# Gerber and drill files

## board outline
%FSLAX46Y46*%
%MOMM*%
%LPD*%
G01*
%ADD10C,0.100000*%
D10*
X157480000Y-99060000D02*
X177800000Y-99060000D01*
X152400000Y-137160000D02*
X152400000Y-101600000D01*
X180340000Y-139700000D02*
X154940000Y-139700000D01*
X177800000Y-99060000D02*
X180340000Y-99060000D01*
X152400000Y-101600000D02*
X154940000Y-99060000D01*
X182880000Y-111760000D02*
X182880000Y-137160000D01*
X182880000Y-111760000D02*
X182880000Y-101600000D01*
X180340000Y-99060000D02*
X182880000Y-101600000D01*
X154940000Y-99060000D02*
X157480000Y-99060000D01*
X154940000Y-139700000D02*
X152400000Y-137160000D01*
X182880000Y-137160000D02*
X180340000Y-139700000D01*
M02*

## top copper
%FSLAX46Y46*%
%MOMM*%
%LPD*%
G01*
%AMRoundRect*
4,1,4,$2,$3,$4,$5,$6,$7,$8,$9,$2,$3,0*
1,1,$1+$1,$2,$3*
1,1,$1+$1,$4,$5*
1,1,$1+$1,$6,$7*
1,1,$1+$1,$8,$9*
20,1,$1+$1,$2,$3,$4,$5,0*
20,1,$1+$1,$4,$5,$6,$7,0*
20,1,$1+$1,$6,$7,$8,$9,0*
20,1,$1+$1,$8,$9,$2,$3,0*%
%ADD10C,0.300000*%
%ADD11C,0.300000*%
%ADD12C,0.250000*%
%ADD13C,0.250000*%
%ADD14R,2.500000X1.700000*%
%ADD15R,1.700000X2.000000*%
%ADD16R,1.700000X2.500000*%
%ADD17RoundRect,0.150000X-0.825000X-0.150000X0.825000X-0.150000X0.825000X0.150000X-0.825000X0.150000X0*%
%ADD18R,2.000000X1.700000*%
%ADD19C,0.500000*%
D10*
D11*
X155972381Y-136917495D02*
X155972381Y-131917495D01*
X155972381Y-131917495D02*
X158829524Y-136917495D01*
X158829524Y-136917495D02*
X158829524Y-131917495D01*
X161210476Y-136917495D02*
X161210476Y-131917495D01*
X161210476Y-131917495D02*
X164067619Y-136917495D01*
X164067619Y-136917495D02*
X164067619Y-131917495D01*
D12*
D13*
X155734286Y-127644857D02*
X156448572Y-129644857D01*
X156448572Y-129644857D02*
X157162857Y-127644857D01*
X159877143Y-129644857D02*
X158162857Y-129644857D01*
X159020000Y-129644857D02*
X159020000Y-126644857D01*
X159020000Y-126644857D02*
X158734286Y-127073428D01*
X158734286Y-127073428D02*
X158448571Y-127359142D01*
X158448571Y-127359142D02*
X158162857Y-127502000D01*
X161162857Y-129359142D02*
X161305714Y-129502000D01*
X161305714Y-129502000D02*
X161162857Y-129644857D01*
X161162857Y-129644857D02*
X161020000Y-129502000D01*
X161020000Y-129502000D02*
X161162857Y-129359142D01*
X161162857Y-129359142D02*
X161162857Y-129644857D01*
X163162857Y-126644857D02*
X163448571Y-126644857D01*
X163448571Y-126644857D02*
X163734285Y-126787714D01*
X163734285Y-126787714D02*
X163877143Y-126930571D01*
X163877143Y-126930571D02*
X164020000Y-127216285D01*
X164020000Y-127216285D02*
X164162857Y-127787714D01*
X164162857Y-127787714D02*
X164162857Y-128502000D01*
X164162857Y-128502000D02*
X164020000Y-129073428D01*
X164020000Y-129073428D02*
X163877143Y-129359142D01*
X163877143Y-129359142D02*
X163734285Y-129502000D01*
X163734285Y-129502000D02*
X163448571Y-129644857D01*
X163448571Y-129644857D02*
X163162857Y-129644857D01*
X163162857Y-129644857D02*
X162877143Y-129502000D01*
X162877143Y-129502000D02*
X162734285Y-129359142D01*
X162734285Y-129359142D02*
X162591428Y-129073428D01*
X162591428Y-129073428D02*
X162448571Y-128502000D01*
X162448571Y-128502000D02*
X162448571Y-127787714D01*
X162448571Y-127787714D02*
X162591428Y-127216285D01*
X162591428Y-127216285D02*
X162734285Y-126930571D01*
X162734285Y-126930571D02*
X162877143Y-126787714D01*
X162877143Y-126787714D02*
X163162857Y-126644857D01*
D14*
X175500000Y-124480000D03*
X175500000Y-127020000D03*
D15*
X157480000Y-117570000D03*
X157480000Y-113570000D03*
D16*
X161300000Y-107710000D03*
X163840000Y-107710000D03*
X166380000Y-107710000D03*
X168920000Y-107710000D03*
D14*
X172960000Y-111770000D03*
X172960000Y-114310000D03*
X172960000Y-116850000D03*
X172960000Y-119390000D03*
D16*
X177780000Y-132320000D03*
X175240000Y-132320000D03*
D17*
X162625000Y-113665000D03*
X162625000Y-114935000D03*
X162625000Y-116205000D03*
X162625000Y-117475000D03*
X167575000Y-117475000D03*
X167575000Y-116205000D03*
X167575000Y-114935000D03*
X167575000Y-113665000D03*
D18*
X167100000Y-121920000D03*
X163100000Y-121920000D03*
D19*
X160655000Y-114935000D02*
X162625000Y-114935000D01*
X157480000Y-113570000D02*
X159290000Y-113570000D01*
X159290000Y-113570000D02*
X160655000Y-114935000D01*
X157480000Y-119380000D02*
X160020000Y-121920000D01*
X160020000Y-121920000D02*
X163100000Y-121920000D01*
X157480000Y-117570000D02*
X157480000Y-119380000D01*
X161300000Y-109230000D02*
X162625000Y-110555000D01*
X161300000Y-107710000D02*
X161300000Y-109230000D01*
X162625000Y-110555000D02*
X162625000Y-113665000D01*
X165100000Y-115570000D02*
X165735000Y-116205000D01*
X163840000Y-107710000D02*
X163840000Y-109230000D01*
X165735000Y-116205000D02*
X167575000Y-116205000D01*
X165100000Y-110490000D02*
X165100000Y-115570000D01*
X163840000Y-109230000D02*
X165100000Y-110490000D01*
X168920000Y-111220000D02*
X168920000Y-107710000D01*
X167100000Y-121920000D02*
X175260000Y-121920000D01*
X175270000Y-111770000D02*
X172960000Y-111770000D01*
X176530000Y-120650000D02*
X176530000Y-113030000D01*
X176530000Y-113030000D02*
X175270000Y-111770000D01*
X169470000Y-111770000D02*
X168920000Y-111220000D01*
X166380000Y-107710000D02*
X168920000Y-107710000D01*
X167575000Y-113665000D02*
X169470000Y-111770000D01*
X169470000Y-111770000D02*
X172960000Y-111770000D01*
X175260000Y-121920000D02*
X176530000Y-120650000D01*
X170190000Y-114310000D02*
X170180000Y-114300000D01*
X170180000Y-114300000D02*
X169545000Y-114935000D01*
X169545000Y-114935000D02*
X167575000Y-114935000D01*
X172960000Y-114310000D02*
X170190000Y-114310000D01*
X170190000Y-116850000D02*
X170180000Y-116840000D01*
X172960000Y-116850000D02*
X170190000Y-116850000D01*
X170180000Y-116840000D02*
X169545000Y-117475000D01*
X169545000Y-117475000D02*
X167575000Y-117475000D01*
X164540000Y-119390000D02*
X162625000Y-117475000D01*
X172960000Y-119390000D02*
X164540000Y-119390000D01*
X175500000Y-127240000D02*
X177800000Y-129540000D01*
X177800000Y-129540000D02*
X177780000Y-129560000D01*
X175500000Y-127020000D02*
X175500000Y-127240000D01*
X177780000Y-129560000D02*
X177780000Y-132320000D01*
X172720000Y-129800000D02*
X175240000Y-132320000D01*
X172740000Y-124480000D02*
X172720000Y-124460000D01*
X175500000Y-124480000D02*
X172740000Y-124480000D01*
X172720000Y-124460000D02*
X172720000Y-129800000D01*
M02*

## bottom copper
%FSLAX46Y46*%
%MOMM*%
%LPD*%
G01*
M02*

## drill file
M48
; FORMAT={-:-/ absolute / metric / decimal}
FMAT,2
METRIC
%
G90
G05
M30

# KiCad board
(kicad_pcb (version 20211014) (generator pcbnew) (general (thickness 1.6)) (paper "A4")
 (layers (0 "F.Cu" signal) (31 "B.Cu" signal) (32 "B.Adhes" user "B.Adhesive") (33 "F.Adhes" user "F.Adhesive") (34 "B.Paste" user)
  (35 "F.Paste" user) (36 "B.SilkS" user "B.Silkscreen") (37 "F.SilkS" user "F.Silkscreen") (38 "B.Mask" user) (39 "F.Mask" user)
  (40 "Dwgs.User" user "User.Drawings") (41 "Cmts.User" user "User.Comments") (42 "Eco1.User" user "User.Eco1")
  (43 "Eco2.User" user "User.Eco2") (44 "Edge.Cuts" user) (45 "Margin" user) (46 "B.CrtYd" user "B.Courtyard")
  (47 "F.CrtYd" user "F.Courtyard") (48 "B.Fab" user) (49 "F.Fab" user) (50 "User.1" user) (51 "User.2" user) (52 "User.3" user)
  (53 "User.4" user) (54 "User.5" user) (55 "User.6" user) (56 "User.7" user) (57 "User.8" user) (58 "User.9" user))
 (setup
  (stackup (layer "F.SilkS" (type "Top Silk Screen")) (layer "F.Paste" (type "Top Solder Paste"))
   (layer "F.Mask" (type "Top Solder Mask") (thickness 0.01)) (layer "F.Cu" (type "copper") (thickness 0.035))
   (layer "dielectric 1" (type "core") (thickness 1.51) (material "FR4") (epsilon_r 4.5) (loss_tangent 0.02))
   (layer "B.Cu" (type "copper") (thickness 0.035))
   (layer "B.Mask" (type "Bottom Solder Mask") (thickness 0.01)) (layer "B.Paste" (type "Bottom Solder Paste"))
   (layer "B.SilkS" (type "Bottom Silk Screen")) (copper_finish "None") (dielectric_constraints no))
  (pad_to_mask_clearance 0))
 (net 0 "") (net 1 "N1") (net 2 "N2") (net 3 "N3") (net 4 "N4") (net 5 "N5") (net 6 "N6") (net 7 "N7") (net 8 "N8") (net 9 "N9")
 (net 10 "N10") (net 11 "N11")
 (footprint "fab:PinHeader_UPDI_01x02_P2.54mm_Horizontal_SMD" (layer "F.Cu") (at 175.5 124.48)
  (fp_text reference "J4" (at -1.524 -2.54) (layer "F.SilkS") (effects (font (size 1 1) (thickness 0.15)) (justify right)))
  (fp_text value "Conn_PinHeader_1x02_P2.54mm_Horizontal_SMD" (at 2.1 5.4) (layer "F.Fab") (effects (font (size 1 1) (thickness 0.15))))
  (pad "1" smd rect locked (at 0 0) (size 2.5 1.7) (layers "F.Cu" "F.Paste" "F.Mask") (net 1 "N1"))
  (pad "2" smd rect locked (at 0 2.54) (size 2.5 1.7) (layers "F.Cu" "F.Paste" "F.Mask") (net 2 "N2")))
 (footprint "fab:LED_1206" (layer "F.Cu") (at 157.48 115.57 90)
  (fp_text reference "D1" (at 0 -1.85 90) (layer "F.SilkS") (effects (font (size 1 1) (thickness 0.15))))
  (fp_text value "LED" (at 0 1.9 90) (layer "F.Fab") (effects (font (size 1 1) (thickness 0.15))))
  (pad "1" smd rect locked (at -2 0 90) (size 2 1.7) (layers "F.Cu" "F.Paste" "F.Mask") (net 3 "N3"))
  (pad "2" smd rect locked (at 2 0 90) (size 2 1.7) (layers "F.Cu" "F.Paste" "F.Mask") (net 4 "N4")))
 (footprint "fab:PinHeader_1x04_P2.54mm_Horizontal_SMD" (layer "F.Cu") (at 161.3 107.71 90)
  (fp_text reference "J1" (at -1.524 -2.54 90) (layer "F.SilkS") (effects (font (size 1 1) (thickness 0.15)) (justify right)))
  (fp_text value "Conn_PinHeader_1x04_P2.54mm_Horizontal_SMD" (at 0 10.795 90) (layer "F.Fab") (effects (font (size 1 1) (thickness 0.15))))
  (pad "1" smd rect locked (at 0 0 90) (size 2.5 1.7) (layers "F.Cu" "F.Paste" "F.Mask") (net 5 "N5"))
  (pad "2" smd rect locked (at 0 2.54 90) (size 2.5 1.7) (layers "F.Cu" "F.Paste" "F.Mask") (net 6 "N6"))
  (pad "3" smd rect locked (at 0 5.08 90) (size 2.5 1.7) (layers "F.Cu" "F.Paste" "F.Mask") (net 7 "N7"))
  (pad "4" smd rect locked (at 0 7.62 90) (size 2.5 1.7) (layers "F.Cu" "F.Paste" "F.Mask") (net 7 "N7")))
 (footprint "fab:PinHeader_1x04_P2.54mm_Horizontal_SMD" (layer "F.Cu") (at 172.96 111.77)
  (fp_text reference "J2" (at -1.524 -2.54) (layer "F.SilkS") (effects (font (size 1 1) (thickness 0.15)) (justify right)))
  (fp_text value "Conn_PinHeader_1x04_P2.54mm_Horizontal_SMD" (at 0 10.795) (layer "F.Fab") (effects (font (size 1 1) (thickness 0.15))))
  (pad "1" smd rect locked (at 0 0) (size 2.5 1.7) (layers "F.Cu" "F.Paste" "F.Mask") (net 7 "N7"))
  (pad "2" smd rect locked (at 0 2.54) (size 2.5 1.7) (layers "F.Cu" "F.Paste" "F.Mask") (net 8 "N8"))
  (pad "3" smd rect locked (at 0 5.08) (size 2.5 1.7) (layers "F.Cu" "F.Paste" "F.Mask") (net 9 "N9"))
  (pad "4" smd rect locked (at 0 7.62) (size 2.5 1.7) (layers "F.Cu" "F.Paste" "F.Mask") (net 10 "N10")))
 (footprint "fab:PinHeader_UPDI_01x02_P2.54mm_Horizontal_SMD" (layer "F.Cu") (at 177.78 132.32 -90)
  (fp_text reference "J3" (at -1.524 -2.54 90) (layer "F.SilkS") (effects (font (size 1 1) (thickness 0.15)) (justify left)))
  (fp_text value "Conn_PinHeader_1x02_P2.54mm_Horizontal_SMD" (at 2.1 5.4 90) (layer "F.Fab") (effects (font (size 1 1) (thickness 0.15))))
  (pad "1" smd rect locked (at 0 0 270) (size 2.5 1.7) (layers "F.Cu" "F.Paste" "F.Mask") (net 2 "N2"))
  (pad "2" smd rect locked (at 0 2.54 270) (size 2.5 1.7) (layers "F.Cu" "F.Paste" "F.Mask") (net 1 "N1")))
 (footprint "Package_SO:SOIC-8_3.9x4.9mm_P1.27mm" (layer "F.Cu") (at 165.1 115.57)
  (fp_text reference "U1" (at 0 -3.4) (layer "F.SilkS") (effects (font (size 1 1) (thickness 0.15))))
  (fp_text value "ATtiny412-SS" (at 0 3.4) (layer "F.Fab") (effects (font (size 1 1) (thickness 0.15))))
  (pad "1" smd roundrect (at -2.475 -1.905) (size 1.95 0.6) (layers "F.Cu" "F.Paste" "F.Mask") (roundrect_rratio 0.25) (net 5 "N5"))
  (pad "2" smd roundrect (at -2.475 -0.635) (size 1.95 0.6) (layers "F.Cu" "F.Paste" "F.Mask") (roundrect_rratio 0.25) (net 4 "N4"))
  (pad "3" smd roundrect (at -2.475 0.635) (size 1.95 0.6) (layers "F.Cu" "F.Paste" "F.Mask") (roundrect_rratio 0.25) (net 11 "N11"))
  (pad "4" smd roundrect (at -2.475 1.905) (size 1.95 0.6) (layers "F.Cu" "F.Paste" "F.Mask") (roundrect_rratio 0.25) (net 10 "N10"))
  (pad "5" smd roundrect (at 2.475 1.905) (size 1.95 0.6) (layers "F.Cu" "F.Paste" "F.Mask") (roundrect_rratio 0.25) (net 9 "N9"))
  (pad "6" smd roundrect (at 2.475 0.635) (size 1.95 0.6) (layers "F.Cu" "F.Paste" "F.Mask") (roundrect_rratio 0.25) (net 6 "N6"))
  (pad "7" smd roundrect (at 2.475 -0.635) (size 1.95 0.6) (layers "F.Cu" "F.Paste" "F.Mask") (roundrect_rratio 0.25) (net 8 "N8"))
  (pad "8" smd roundrect (at 2.475 -1.905) (size 1.95 0.6) (layers "F.Cu" "F.Paste" "F.Mask") (roundrect_rratio 0.25) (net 7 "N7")))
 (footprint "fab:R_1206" (layer "F.Cu") (at 165.1 121.92 180)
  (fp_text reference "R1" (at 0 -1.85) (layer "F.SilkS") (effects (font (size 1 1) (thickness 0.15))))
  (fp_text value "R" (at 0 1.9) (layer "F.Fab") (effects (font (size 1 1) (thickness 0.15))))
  (pad "1" smd rect locked (at -2 0 180) (size 2 1.7) (layers "F.Cu" "F.Paste" "F.Mask") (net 7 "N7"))
  (pad "2" smd rect locked (at 2 0 180) (size 2 1.7) (layers "F.Cu" "F.Paste" "F.Mask") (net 3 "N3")))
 (gr_line (start 157.48 99.06) (end 177.8 99.06) (layer "Edge.Cuts") (width 0.1))
 (gr_line (start 152.4 137.16) (end 152.4 101.6) (layer "Edge.Cuts") (width 0.1))
 (gr_line (start 180.34 139.7) (end 154.94 139.7) (layer "Edge.Cuts") (width 0.1))
 (gr_line (start 177.8 99.06) (end 180.34 99.06) (layer "Edge.Cuts") (width 0.1))
 (gr_line (start 152.4 101.6) (end 154.94 99.06) (layer "Edge.Cuts") (width 0.1))
 (gr_line (start 182.88 111.76) (end 182.88 137.16) (layer "Edge.Cuts") (width 0.1))
 (gr_line (start 182.88 111.76) (end 182.88 101.6) (layer "Edge.Cuts") (width 0.1))
 (gr_line (start 180.34 99.06) (end 182.88 101.6) (layer "Edge.Cuts") (width 0.1))
 (gr_line (start 154.94 99.06) (end 157.48 99.06) (layer "Edge.Cuts") (width 0.1))
 (gr_line (start 154.94 139.7) (end 152.4 137.16) (layer "Edge.Cuts") (width 0.1))
 (gr_line (start 182.88 137.16) (end 180.34 139.7) (layer "Edge.Cuts") (width 0.1))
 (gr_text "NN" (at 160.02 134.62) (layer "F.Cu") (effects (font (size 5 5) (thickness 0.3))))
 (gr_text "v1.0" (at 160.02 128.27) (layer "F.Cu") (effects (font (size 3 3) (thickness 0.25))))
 (segment (start 160.655 114.935) (end 162.625 114.935) (width 0.5) (layer "F.Cu") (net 4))
 (segment (start 157.48 113.57) (end 159.29 113.57) (width 0.5) (layer "F.Cu") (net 4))
 (segment (start 159.29 113.57) (end 160.655 114.935) (width 0.5) (layer "F.Cu") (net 4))
 (segment (start 157.48 119.38) (end 160.02 121.92) (width 0.5) (layer "F.Cu") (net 3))
 (segment (start 160.02 121.92) (end 163.1 121.92) (width 0.5) (layer "F.Cu") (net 3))
 (segment (start 157.48 117.57) (end 157.48 119.38) (width 0.5) (layer "F.Cu") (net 3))
 (segment (start 161.3 109.23) (end 162.625 110.555) (width 0.5) (layer "F.Cu") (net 5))
 (segment (start 161.3 107.71) (end 161.3 109.23) (width 0.5) (layer "F.Cu") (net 5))
 (segment (start 162.625 110.555) (end 162.625 113.665) (width 0.5) (layer "F.Cu") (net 5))
 (segment (start 165.1 115.57) (end 165.735 116.205) (width 0.5) (layer "F.Cu") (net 6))
 (segment (start 163.84 107.71) (end 163.84 109.23) (width 0.5) (layer "F.Cu") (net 6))
 (segment (start 165.735 116.205) (end 167.575 116.205) (width 0.5) (layer "F.Cu") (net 6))
 (segment (start 165.1 110.49) (end 165.1 115.57) (width 0.5) (layer "F.Cu") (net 6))
 (segment (start 163.84 109.23) (end 165.1 110.49) (width 0.5) (layer "F.Cu") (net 6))
 (segment (start 168.92 111.22) (end 168.92 107.71) (width 0.5) (layer "F.Cu") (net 7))
 (segment (start 167.1 121.92) (end 175.26 121.92) (width 0.5) (layer "F.Cu") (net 7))
 (segment (start 175.27 111.77) (end 172.96 111.77) (width 0.5) (layer "F.Cu") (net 7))
 (segment (start 176.53 120.65) (end 176.53 113.03) (width 0.5) (layer "F.Cu") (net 7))
 (segment (start 176.53 113.03) (end 175.27 111.77) (width 0.5) (layer "F.Cu") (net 7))
 (segment (start 169.47 111.77) (end 168.92 111.22) (width 0.5) (layer "F.Cu") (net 7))
 (segment (start 166.38 107.71) (end 168.92 107.71) (width 0.5) (layer "F.Cu") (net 7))
 (segment (start 167.575 113.665) (end 169.47 111.77) (width 0.5) (layer "F.Cu") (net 7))
 (segment (start 169.47 111.77) (end 172.96 111.77) (width 0.5) (layer "F.Cu") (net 7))
 (segment (start 175.26 121.92) (end 176.53 120.65) (width 0.5) (layer "F.Cu") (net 7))
 (segment (start 170.19 114.31) (end 170.18 114.3) (width 0.5) (layer "F.Cu") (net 8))
 (segment (start 170.18 114.3) (end 169.545 114.935) (width 0.5) (layer "F.Cu") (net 8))
 (segment (start 169.545 114.935) (end 167.575 114.935) (width 0.5) (layer "F.Cu") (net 8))
 (segment (start 172.96 114.31) (end 170.19 114.31) (width 0.5) (layer "F.Cu") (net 8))
 (segment (start 170.19 116.85) (end 170.18 116.84) (width 0.5) (layer "F.Cu") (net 9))
 (segment (start 172.96 116.85) (end 170.19 116.85) (width 0.5) (layer "F.Cu") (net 9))
 (segment (start 170.18 116.84) (end 169.545 117.475) (width 0.5) (layer "F.Cu") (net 9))
 (segment (start 169.545 117.475) (end 167.575 117.475) (width 0.5) (layer "F.Cu") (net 9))
 (segment (start 164.54 119.39) (end 162.625 117.475) (width 0.5) (layer "F.Cu") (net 10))
 (segment (start 172.96 119.39) (end 164.54 119.39) (width 0.5) (layer "F.Cu") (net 10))
 (segment (start 175.5 127.24) (end 177.8 129.54) (width 0.5) (layer "F.Cu") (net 2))
 (segment (start 177.8 129.54) (end 177.78 129.56) (width 0.5) (layer "F.Cu") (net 2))
 (segment (start 175.5 127.02) (end 175.5 127.24) (width 0.5) (layer "F.Cu") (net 2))
 (segment (start 177.78 129.56) (end 177.78 132.32) (width 0.5) (layer "F.Cu") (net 2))
 (segment (start 172.72 129.8) (end 175.24 132.32) (width 0.5) (layer "F.Cu") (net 1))
 (segment (start 172.74 124.48) (end 172.72 124.46) (width 0.5) (layer "F.Cu") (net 1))
 (segment (start 175.5 124.48) (end 172.74 124.48) (width 0.5) (layer "F.Cu") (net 1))
 (segment (start 172.72 124.46) (end 172.72 129.8) (width 0.5) (layer "F.Cu") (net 1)))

